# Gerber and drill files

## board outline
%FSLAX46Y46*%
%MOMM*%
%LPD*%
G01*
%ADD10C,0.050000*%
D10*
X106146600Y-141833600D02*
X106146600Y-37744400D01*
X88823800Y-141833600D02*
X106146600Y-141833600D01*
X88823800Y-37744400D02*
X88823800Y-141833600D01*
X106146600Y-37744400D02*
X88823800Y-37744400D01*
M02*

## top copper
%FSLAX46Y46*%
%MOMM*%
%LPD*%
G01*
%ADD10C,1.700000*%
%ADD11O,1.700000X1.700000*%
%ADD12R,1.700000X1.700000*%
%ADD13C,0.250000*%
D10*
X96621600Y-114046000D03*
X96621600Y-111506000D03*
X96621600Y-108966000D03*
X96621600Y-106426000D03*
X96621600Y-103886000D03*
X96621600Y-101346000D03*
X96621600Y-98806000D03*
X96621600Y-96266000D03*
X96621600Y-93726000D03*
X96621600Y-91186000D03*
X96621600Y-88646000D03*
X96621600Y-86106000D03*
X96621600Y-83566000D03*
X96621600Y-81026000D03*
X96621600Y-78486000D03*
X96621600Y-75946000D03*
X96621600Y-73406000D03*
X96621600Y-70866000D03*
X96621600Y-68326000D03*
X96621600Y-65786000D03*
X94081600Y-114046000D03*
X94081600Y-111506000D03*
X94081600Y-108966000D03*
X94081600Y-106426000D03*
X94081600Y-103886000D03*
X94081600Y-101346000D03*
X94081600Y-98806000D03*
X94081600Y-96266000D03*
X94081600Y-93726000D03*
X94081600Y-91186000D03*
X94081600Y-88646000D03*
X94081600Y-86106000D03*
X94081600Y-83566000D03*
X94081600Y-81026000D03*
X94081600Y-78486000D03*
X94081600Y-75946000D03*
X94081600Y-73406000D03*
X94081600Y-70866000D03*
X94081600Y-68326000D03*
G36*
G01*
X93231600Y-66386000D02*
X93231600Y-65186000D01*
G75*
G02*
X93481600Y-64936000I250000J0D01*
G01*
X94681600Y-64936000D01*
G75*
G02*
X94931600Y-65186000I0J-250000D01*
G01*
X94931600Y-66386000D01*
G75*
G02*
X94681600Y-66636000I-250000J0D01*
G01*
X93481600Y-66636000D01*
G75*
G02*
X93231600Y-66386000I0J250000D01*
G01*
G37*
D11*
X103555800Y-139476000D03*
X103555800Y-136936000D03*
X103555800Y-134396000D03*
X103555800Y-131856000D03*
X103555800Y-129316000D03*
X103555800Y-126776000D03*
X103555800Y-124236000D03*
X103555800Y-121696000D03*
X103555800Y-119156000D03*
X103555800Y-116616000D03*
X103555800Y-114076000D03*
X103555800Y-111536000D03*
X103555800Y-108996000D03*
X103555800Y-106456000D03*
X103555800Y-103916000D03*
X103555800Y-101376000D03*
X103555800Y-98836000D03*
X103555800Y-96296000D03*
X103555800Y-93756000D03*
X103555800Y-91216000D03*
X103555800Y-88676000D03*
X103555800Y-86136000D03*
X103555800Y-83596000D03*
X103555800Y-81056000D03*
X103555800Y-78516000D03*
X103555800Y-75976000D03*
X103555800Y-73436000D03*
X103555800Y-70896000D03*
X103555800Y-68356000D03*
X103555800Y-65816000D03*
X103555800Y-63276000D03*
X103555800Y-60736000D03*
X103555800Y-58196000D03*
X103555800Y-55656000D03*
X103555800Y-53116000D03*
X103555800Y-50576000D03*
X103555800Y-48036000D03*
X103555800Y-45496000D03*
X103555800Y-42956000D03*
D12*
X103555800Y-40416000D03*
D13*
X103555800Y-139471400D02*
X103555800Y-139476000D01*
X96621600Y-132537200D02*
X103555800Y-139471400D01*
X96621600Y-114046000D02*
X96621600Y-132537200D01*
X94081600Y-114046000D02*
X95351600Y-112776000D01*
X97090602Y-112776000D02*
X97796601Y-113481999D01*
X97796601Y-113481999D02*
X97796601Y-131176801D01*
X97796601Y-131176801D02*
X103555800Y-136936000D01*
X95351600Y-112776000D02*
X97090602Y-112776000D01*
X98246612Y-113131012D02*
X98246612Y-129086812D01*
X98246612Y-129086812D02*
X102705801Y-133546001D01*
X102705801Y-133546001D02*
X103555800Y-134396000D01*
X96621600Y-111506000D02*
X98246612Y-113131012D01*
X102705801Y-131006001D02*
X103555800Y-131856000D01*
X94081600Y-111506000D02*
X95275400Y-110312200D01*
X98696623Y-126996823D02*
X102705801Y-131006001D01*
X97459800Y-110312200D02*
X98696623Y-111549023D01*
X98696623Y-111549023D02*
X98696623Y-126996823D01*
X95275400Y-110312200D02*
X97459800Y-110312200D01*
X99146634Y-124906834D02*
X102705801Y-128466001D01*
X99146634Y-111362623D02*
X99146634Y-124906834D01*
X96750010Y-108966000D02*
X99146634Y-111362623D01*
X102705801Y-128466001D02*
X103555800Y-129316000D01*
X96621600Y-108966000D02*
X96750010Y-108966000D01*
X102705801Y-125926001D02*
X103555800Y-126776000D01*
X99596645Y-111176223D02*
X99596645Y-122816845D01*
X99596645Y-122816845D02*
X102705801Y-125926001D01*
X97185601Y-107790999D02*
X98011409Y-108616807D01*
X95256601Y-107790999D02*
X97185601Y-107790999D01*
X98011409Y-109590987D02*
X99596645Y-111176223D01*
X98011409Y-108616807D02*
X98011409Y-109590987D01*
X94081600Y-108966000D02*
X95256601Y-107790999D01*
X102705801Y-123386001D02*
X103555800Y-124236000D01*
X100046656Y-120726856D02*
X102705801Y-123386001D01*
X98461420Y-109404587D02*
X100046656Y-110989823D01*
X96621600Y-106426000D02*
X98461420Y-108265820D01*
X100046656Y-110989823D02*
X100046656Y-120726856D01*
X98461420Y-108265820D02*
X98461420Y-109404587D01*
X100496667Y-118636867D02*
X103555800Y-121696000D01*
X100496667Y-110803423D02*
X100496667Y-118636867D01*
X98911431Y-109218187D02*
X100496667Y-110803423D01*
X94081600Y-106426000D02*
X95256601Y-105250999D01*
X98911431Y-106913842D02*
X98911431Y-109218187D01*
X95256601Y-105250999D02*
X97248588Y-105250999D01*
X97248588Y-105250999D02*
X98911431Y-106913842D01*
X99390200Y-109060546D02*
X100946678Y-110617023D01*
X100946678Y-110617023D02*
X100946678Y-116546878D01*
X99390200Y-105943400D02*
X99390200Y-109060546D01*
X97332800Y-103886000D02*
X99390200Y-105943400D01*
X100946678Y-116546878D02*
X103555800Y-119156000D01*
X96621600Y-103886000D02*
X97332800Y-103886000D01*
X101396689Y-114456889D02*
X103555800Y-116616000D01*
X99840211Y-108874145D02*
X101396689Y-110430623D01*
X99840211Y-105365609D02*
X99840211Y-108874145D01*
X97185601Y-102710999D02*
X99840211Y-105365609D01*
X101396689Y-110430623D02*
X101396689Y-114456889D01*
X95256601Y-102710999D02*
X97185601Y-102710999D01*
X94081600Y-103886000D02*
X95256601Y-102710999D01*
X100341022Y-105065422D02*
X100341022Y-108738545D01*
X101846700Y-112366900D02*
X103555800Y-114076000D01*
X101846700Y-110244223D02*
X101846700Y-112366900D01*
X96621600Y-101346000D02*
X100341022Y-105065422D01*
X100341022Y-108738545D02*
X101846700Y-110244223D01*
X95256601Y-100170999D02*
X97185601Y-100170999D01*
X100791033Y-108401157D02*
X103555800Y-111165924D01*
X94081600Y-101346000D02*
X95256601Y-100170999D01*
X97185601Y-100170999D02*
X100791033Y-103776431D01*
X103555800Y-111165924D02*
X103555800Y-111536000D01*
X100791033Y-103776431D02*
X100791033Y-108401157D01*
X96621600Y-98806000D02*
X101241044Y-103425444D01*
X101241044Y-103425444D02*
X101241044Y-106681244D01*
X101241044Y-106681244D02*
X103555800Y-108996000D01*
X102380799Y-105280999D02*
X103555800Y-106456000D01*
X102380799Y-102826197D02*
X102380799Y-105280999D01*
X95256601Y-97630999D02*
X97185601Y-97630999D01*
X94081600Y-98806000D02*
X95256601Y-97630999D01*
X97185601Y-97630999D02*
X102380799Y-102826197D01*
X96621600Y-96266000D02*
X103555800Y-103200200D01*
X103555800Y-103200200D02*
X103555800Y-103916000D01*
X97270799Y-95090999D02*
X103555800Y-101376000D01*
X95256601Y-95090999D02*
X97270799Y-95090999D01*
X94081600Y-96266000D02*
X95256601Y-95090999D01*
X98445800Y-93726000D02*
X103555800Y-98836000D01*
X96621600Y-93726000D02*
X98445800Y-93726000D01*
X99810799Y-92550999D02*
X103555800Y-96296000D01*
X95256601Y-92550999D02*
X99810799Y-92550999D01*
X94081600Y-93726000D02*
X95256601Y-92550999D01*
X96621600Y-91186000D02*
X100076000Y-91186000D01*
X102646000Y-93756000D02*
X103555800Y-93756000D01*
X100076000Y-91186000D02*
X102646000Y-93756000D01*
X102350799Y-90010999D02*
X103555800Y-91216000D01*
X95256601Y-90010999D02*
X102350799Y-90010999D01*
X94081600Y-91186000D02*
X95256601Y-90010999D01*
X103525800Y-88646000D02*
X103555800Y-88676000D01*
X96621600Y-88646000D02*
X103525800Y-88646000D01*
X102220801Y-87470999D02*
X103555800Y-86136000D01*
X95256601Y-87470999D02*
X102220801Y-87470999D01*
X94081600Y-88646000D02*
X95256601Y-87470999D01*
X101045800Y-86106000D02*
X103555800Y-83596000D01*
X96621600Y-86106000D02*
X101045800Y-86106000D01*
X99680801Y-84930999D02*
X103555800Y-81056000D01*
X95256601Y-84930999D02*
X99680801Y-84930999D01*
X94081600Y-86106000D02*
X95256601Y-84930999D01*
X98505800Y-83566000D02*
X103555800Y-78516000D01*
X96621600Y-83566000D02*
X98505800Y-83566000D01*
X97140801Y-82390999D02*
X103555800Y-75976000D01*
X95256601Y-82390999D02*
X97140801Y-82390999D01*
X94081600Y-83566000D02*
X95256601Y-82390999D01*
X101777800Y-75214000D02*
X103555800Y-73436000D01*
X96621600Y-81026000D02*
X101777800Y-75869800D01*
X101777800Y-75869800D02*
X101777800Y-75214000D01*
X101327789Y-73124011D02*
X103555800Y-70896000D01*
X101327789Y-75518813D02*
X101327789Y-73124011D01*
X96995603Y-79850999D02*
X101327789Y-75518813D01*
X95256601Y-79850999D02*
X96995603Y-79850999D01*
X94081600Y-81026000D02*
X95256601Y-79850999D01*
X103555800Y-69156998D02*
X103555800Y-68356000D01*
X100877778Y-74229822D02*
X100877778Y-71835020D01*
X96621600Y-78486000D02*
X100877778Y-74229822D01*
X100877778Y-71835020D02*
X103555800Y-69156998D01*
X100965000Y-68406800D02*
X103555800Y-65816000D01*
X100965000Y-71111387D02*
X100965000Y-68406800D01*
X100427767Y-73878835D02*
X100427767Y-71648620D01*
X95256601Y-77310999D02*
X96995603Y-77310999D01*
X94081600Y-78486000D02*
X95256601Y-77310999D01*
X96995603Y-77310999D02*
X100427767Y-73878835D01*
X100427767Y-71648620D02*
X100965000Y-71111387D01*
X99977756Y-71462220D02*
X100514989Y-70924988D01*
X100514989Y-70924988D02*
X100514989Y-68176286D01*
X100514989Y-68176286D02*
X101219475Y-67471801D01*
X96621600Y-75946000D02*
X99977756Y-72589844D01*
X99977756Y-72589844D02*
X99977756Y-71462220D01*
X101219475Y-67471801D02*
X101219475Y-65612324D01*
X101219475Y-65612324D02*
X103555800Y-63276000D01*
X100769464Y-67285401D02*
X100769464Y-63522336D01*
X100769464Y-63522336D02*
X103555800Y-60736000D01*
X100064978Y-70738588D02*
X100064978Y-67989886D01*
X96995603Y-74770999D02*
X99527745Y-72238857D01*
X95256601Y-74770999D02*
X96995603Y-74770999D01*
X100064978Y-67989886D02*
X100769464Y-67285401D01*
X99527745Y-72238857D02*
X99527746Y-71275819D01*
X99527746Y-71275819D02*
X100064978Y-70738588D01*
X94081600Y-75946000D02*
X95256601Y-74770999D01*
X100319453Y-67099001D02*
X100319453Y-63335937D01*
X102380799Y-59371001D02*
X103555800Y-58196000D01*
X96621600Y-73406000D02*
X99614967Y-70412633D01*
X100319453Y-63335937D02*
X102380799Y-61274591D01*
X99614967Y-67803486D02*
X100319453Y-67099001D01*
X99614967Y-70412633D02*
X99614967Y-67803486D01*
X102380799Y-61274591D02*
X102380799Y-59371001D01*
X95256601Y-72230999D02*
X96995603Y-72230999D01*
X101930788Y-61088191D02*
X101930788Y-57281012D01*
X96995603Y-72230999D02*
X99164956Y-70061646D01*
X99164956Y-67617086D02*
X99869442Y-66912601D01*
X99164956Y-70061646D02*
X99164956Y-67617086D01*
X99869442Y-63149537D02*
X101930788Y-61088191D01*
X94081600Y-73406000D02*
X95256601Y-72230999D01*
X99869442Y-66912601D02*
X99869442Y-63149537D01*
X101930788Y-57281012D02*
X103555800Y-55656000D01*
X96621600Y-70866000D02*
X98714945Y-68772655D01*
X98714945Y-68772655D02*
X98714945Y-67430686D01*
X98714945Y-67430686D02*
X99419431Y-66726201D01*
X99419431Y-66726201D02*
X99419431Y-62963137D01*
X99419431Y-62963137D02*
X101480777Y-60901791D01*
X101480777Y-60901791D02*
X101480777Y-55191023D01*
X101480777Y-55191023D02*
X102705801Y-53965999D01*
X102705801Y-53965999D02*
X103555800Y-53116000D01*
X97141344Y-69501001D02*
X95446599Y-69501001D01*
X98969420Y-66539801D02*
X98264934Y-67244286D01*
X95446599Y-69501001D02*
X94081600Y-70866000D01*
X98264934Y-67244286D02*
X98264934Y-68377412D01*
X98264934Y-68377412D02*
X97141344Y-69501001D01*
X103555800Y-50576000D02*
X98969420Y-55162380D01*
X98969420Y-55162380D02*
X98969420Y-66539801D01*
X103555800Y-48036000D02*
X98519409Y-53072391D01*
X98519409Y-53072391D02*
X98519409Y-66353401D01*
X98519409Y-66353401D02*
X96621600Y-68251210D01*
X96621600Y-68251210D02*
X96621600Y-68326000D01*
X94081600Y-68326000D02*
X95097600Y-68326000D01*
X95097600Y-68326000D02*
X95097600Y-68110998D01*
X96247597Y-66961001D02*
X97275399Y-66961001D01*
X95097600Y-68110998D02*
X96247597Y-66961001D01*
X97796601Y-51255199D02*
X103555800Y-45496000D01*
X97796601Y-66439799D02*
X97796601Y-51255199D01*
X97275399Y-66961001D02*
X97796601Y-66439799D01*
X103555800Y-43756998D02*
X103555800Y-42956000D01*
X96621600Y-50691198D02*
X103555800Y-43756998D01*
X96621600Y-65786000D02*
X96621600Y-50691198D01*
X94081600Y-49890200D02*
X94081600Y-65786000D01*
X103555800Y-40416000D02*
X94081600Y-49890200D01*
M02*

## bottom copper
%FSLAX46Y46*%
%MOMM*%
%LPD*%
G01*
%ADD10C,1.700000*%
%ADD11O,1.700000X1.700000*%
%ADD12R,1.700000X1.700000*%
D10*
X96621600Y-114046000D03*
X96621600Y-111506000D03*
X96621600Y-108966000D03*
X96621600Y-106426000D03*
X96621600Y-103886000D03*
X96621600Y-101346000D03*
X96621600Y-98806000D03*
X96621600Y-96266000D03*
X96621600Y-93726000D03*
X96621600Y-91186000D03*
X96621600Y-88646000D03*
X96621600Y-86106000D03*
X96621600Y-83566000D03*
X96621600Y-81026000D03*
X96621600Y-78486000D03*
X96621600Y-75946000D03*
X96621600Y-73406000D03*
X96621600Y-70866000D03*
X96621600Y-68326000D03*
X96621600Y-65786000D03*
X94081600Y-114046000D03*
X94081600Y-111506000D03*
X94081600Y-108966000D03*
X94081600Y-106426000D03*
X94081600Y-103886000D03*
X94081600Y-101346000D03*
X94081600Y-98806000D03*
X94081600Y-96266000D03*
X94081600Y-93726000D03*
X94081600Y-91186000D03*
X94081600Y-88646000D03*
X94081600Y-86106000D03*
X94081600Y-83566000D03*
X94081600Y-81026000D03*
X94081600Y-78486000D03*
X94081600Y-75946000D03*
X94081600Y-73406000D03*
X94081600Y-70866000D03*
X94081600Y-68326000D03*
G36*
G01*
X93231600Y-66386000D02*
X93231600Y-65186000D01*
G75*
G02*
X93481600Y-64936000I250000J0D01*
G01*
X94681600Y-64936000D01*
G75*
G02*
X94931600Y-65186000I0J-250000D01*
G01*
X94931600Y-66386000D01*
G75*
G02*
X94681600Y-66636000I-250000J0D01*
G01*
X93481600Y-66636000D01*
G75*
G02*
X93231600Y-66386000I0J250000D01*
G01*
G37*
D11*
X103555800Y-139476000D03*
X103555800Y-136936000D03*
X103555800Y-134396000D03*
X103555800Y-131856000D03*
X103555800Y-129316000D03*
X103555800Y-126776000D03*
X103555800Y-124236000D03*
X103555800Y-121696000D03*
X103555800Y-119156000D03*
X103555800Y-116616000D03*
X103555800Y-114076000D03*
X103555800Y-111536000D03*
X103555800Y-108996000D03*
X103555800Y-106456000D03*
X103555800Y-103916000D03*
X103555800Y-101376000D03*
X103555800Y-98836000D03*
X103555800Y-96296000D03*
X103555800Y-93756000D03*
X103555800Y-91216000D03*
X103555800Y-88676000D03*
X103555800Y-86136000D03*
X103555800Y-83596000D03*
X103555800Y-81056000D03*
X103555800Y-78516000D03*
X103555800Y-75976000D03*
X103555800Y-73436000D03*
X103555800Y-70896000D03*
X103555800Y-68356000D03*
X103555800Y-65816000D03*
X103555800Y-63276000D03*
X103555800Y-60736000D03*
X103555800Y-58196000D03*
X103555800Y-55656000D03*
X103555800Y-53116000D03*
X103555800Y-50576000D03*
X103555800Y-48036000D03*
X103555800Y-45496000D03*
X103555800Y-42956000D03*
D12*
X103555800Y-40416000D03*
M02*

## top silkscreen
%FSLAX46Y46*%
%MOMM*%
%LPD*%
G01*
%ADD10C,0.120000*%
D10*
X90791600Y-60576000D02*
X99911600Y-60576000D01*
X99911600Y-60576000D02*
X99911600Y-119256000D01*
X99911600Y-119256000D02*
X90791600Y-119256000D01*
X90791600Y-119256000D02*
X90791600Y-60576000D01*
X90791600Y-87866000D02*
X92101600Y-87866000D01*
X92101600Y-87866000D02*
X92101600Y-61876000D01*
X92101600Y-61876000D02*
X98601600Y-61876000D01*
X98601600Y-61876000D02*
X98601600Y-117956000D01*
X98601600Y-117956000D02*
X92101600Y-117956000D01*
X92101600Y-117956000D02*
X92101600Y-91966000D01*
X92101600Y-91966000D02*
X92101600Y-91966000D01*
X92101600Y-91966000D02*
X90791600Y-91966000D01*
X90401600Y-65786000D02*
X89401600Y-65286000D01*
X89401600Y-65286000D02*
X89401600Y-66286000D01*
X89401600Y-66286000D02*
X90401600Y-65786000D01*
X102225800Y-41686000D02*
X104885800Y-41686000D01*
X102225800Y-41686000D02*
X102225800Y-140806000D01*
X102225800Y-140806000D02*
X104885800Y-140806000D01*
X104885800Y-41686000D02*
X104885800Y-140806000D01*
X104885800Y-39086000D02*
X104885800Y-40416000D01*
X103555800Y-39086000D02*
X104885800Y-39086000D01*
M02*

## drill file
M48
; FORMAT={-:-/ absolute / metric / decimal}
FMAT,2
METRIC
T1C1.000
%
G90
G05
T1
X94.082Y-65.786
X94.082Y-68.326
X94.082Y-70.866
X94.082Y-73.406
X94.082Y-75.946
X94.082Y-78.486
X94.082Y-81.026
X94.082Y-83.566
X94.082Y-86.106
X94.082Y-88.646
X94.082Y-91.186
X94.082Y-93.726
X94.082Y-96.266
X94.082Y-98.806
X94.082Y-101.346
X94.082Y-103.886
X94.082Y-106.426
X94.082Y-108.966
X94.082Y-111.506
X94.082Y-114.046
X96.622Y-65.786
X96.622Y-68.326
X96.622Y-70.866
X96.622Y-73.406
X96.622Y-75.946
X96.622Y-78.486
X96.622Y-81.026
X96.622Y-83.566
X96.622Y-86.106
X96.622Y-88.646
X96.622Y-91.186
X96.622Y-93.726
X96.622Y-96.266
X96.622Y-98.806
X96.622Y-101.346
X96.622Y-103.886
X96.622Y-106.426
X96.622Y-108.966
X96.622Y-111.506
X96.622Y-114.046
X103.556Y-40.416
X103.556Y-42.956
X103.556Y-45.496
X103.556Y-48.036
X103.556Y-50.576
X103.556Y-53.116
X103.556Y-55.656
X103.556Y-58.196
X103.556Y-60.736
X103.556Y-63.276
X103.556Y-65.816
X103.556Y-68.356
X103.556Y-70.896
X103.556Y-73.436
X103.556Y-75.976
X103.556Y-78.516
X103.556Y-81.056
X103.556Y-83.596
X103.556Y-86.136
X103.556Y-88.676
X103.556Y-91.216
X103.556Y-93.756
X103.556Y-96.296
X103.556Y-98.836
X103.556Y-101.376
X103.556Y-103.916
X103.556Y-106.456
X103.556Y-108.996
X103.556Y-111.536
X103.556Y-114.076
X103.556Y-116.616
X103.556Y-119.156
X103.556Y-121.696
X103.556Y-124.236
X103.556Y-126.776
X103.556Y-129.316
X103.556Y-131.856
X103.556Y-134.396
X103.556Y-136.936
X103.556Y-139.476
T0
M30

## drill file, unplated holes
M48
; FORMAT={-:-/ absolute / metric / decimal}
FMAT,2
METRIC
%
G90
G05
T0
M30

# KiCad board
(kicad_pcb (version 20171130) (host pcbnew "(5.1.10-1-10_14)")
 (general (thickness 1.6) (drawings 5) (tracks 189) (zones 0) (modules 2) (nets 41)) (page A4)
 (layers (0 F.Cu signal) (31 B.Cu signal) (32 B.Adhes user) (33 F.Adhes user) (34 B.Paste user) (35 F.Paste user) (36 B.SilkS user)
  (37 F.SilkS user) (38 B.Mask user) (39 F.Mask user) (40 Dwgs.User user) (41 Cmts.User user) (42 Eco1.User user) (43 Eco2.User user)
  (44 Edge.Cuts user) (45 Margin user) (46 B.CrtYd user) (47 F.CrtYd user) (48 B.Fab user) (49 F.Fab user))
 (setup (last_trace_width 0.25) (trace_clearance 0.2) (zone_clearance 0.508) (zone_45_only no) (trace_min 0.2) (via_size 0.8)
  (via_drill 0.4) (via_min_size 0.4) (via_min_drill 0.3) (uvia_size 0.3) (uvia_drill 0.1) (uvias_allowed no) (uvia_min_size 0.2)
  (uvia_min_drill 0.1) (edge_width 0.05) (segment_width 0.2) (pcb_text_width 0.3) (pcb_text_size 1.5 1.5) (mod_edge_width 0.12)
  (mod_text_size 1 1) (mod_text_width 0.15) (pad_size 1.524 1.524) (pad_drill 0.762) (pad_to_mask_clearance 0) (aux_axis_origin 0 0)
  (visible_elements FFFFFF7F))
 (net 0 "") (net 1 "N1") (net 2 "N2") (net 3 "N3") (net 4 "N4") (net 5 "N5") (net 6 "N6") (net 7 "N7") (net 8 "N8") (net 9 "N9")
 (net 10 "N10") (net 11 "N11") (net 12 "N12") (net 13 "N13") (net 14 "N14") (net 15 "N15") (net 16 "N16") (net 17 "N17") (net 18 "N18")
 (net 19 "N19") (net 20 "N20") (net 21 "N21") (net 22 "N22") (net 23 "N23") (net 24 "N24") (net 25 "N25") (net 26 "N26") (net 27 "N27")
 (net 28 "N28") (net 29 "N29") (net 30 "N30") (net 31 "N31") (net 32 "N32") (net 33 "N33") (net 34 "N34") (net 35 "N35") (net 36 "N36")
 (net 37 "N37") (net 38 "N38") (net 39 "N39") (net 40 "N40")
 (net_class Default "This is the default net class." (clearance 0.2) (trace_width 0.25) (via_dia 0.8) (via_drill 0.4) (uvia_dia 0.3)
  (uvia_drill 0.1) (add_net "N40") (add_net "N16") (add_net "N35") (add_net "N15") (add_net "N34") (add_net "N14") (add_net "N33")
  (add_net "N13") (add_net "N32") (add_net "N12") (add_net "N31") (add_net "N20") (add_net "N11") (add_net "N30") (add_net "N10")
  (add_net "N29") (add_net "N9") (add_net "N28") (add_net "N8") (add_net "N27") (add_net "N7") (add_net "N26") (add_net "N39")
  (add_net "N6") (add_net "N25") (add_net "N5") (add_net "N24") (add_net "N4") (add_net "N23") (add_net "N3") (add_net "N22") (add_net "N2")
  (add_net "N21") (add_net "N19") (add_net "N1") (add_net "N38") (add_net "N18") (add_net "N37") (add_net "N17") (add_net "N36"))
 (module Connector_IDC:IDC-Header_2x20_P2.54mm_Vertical (layer F.Cu) (at 94.0816 65.786)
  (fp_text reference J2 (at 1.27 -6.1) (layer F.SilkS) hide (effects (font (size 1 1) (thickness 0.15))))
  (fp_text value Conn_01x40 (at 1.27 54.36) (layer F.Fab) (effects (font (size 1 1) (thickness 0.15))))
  (fp_line (start -3.29 -5.21) (end 5.83 -5.21) (layer F.SilkS) (width 0.12))
  (fp_line (start 5.83 -5.21) (end 5.83 53.47) (layer F.SilkS) (width 0.12))
  (fp_line (start 5.83 53.47) (end -3.29 53.47) (layer F.SilkS) (width 0.12))
  (fp_line (start -3.29 53.47) (end -3.29 -5.21) (layer F.SilkS) (width 0.12))
  (fp_line (start -3.29 22.08) (end -1.98 22.08) (layer F.SilkS) (width 0.12))
  (fp_line (start -1.98 22.08) (end -1.98 -3.91) (layer F.SilkS) (width 0.12))
  (fp_line (start -1.98 -3.91) (end 4.52 -3.91) (layer F.SilkS) (width 0.12))
  (fp_line (start 4.52 -3.91) (end 4.52 52.17) (layer F.SilkS) (width 0.12))
  (fp_line (start 4.52 52.17) (end -1.98 52.17) (layer F.SilkS) (width 0.12))
  (fp_line (start -1.98 52.17) (end -1.98 26.18) (layer F.SilkS) (width 0.12))
  (fp_line (start -1.98 26.18) (end -1.98 26.18) (layer F.SilkS) (width 0.12))
  (fp_line (start -1.98 26.18) (end -3.29 26.18) (layer F.SilkS) (width 0.12))
  (fp_line (start -3.68 0) (end -4.68 -0.5) (layer F.SilkS) (width 0.12))
  (fp_line (start -4.68 -0.5) (end -4.68 0.5) (layer F.SilkS) (width 0.12))
  (fp_line (start -4.68 0.5) (end -3.68 0) (layer F.SilkS) (width 0.12))
  (pad 40 thru_hole circle (at 2.54 48.26) (size 1.7 1.7) (drill 1) (layers *.Cu *.Mask) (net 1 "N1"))
  (pad 38 thru_hole circle (at 2.54 45.72) (size 1.7 1.7) (drill 1) (layers *.Cu *.Mask) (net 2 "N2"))
  (pad 36 thru_hole circle (at 2.54 43.18) (size 1.7 1.7) (drill 1) (layers *.Cu *.Mask) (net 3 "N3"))
  (pad 34 thru_hole circle (at 2.54 40.64) (size 1.7 1.7) (drill 1) (layers *.Cu *.Mask) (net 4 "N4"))
  (pad 32 thru_hole circle (at 2.54 38.1) (size 1.7 1.7) (drill 1) (layers *.Cu *.Mask) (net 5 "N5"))
  (pad 30 thru_hole circle (at 2.54 35.56) (size 1.7 1.7) (drill 1) (layers *.Cu *.Mask) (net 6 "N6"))
  (pad 28 thru_hole circle (at 2.54 33.02) (size 1.7 1.7) (drill 1) (layers *.Cu *.Mask) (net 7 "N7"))
  (pad 26 thru_hole circle (at 2.54 30.48) (size 1.7 1.7) (drill 1) (layers *.Cu *.Mask) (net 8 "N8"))
  (pad 24 thru_hole circle (at 2.54 27.94) (size 1.7 1.7) (drill 1) (layers *.Cu *.Mask) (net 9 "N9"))
  (pad 22 thru_hole circle (at 2.54 25.4) (size 1.7 1.7) (drill 1) (layers *.Cu *.Mask) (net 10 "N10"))
  (pad 20 thru_hole circle (at 2.54 22.86) (size 1.7 1.7) (drill 1) (layers *.Cu *.Mask) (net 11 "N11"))
  (pad 18 thru_hole circle (at 2.54 20.32) (size 1.7 1.7) (drill 1) (layers *.Cu *.Mask) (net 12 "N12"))
  (pad 16 thru_hole circle (at 2.54 17.78) (size 1.7 1.7) (drill 1) (layers *.Cu *.Mask) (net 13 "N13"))
  (pad 14 thru_hole circle (at 2.54 15.24) (size 1.7 1.7) (drill 1) (layers *.Cu *.Mask) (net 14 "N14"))
  (pad 12 thru_hole circle (at 2.54 12.7) (size 1.7 1.7) (drill 1) (layers *.Cu *.Mask) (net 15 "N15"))
  (pad 10 thru_hole circle (at 2.54 10.16) (size 1.7 1.7) (drill 1) (layers *.Cu *.Mask) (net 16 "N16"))
  (pad 8 thru_hole circle (at 2.54 7.62) (size 1.7 1.7) (drill 1) (layers *.Cu *.Mask) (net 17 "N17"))
  (pad 6 thru_hole circle (at 2.54 5.08) (size 1.7 1.7) (drill 1) (layers *.Cu *.Mask) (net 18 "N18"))
  (pad 4 thru_hole circle (at 2.54 2.54) (size 1.7 1.7) (drill 1) (layers *.Cu *.Mask) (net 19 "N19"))
  (pad 2 thru_hole circle (at 2.54 0) (size 1.7 1.7) (drill 1) (layers *.Cu *.Mask) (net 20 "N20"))
  (pad 39 thru_hole circle (at 0 48.26) (size 1.7 1.7) (drill 1) (layers *.Cu *.Mask) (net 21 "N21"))
  (pad 37 thru_hole circle (at 0 45.72) (size 1.7 1.7) (drill 1) (layers *.Cu *.Mask) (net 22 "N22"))
  (pad 35 thru_hole circle (at 0 43.18) (size 1.7 1.7) (drill 1) (layers *.Cu *.Mask) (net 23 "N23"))
  (pad 33 thru_hole circle (at 0 40.64) (size 1.7 1.7) (drill 1) (layers *.Cu *.Mask) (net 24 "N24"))
  (pad 31 thru_hole circle (at 0 38.1) (size 1.7 1.7) (drill 1) (layers *.Cu *.Mask) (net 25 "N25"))
  (pad 29 thru_hole circle (at 0 35.56) (size 1.7 1.7) (drill 1) (layers *.Cu *.Mask) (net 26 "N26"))
  (pad 27 thru_hole circle (at 0 33.02) (size 1.7 1.7) (drill 1) (layers *.Cu *.Mask) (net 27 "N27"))
  (pad 25 thru_hole circle (at 0 30.48) (size 1.7 1.7) (drill 1) (layers *.Cu *.Mask) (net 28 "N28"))
  (pad 23 thru_hole circle (at 0 27.94) (size 1.7 1.7) (drill 1) (layers *.Cu *.Mask) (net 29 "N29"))
  (pad 21 thru_hole circle (at 0 25.4) (size 1.7 1.7) (drill 1) (layers *.Cu *.Mask) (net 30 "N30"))
  (pad 19 thru_hole circle (at 0 22.86) (size 1.7 1.7) (drill 1) (layers *.Cu *.Mask) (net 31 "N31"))
  (pad 17 thru_hole circle (at 0 20.32) (size 1.7 1.7) (drill 1) (layers *.Cu *.Mask) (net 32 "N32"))
  (pad 15 thru_hole circle (at 0 17.78) (size 1.7 1.7) (drill 1) (layers *.Cu *.Mask) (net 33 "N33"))
  (pad 13 thru_hole circle (at 0 15.24) (size 1.7 1.7) (drill 1) (layers *.Cu *.Mask) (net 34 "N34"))
  (pad 11 thru_hole circle (at 0 12.7) (size 1.7 1.7) (drill 1) (layers *.Cu *.Mask) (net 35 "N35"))
  (pad 9 thru_hole circle (at 0 10.16) (size 1.7 1.7) (drill 1) (layers *.Cu *.Mask) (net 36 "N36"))
  (pad 7 thru_hole circle (at 0 7.62) (size 1.7 1.7) (drill 1) (layers *.Cu *.Mask) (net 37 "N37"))
  (pad 5 thru_hole circle (at 0 5.08) (size 1.7 1.7) (drill 1) (layers *.Cu *.Mask) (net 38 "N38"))
  (pad 3 thru_hole circle (at 0 2.54) (size 1.7 1.7) (drill 1) (layers *.Cu *.Mask) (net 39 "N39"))
  (pad 1 thru_hole roundrect (at 0 0) (size 1.7 1.7) (drill 1) (layers *.Cu *.Mask) (roundrect_rratio 0.1470588235294118) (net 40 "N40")))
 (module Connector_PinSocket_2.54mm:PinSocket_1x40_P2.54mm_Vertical (layer F.Cu) (at 103.5558 40.416)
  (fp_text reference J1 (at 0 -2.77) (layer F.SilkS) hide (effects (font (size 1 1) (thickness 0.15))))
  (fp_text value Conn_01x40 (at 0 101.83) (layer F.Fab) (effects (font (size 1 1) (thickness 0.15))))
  (fp_line (start -1.33 1.27) (end 1.33 1.27) (layer F.SilkS) (width 0.12))
  (fp_line (start -1.33 1.27) (end -1.33 100.39) (layer F.SilkS) (width 0.12))
  (fp_line (start -1.33 100.39) (end 1.33 100.39) (layer F.SilkS) (width 0.12))
  (fp_line (start 1.33 1.27) (end 1.33 100.39) (layer F.SilkS) (width 0.12))
  (fp_line (start 1.33 -1.33) (end 1.33 0) (layer F.SilkS) (width 0.12))
  (fp_line (start 0 -1.33) (end 1.33 -1.33) (layer F.SilkS) (width 0.12))
  (pad 40 thru_hole oval (at 0 99.06) (size 1.7 1.7) (drill 1) (layers *.Cu *.Mask) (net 1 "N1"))
  (pad 39 thru_hole oval (at 0 96.52) (size 1.7 1.7) (drill 1) (layers *.Cu *.Mask) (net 21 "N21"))
  (pad 38 thru_hole oval (at 0 93.98) (size 1.7 1.7) (drill 1) (layers *.Cu *.Mask) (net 2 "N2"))
  (pad 37 thru_hole oval (at 0 91.44) (size 1.7 1.7) (drill 1) (layers *.Cu *.Mask) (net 22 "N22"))
  (pad 36 thru_hole oval (at 0 88.9) (size 1.7 1.7) (drill 1) (layers *.Cu *.Mask) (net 3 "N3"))
  (pad 35 thru_hole oval (at 0 86.36) (size 1.7 1.7) (drill 1) (layers *.Cu *.Mask) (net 23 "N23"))
  (pad 34 thru_hole oval (at 0 83.82) (size 1.7 1.7) (drill 1) (layers *.Cu *.Mask) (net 4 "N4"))
  (pad 33 thru_hole oval (at 0 81.28) (size 1.7 1.7) (drill 1) (layers *.Cu *.Mask) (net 24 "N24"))
  (pad 32 thru_hole oval (at 0 78.74) (size 1.7 1.7) (drill 1) (layers *.Cu *.Mask) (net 5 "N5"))
  (pad 31 thru_hole oval (at 0 76.2) (size 1.7 1.7) (drill 1) (layers *.Cu *.Mask) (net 25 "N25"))
  (pad 30 thru_hole oval (at 0 73.66) (size 1.7 1.7) (drill 1) (layers *.Cu *.Mask) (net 6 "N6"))
  (pad 29 thru_hole oval (at 0 71.12) (size 1.7 1.7) (drill 1) (layers *.Cu *.Mask) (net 26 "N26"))
  (pad 28 thru_hole oval (at 0 68.58) (size 1.7 1.7) (drill 1) (layers *.Cu *.Mask) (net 7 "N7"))
  (pad 27 thru_hole oval (at 0 66.04) (size 1.7 1.7) (drill 1) (layers *.Cu *.Mask) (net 27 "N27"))
  (pad 26 thru_hole oval (at 0 63.5) (size 1.7 1.7) (drill 1) (layers *.Cu *.Mask) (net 8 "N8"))
  (pad 25 thru_hole oval (at 0 60.96) (size 1.7 1.7) (drill 1) (layers *.Cu *.Mask) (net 28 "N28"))
  (pad 24 thru_hole oval (at 0 58.42) (size 1.7 1.7) (drill 1) (layers *.Cu *.Mask) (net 9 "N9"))
  (pad 23 thru_hole oval (at 0 55.88) (size 1.7 1.7) (drill 1) (layers *.Cu *.Mask) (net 29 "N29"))
  (pad 22 thru_hole oval (at 0 53.34) (size 1.7 1.7) (drill 1) (layers *.Cu *.Mask) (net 10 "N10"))
  (pad 21 thru_hole oval (at 0 50.8) (size 1.7 1.7) (drill 1) (layers *.Cu *.Mask) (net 30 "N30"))
  (pad 20 thru_hole oval (at 0 48.26) (size 1.7 1.7) (drill 1) (layers *.Cu *.Mask) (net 11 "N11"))
  (pad 19 thru_hole oval (at 0 45.72) (size 1.7 1.7) (drill 1) (layers *.Cu *.Mask) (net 31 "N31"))
  (pad 18 thru_hole oval (at 0 43.18) (size 1.7 1.7) (drill 1) (layers *.Cu *.Mask) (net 12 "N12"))
  (pad 17 thru_hole oval (at 0 40.64) (size 1.7 1.7) (drill 1) (layers *.Cu *.Mask) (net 32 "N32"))
  (pad 16 thru_hole oval (at 0 38.1) (size 1.7 1.7) (drill 1) (layers *.Cu *.Mask) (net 13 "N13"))
  (pad 15 thru_hole oval (at 0 35.56) (size 1.7 1.7) (drill 1) (layers *.Cu *.Mask) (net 33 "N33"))
  (pad 14 thru_hole oval (at 0 33.02) (size 1.7 1.7) (drill 1) (layers *.Cu *.Mask) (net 14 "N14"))
  (pad 13 thru_hole oval (at 0 30.48) (size 1.7 1.7) (drill 1) (layers *.Cu *.Mask) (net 34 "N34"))
  (pad 12 thru_hole oval (at 0 27.94) (size 1.7 1.7) (drill 1) (layers *.Cu *.Mask) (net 15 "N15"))
  (pad 11 thru_hole oval (at 0 25.4) (size 1.7 1.7) (drill 1) (layers *.Cu *.Mask) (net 35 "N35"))
  (pad 10 thru_hole oval (at 0 22.86) (size 1.7 1.7) (drill 1) (layers *.Cu *.Mask) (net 16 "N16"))
  (pad 9 thru_hole oval (at 0 20.32) (size 1.7 1.7) (drill 1) (layers *.Cu *.Mask) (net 36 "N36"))
  (pad 8 thru_hole oval (at 0 17.78) (size 1.7 1.7) (drill 1) (layers *.Cu *.Mask) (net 17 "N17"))
  (pad 7 thru_hole oval (at 0 15.24) (size 1.7 1.7) (drill 1) (layers *.Cu *.Mask) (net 37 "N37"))
  (pad 6 thru_hole oval (at 0 12.7) (size 1.7 1.7) (drill 1) (layers *.Cu *.Mask) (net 18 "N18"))
  (pad 5 thru_hole oval (at 0 10.16) (size 1.7 1.7) (drill 1) (layers *.Cu *.Mask) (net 38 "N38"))
  (pad 4 thru_hole oval (at 0 7.62) (size 1.7 1.7) (drill 1) (layers *.Cu *.Mask) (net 19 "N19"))
  (pad 3 thru_hole oval (at 0 5.08) (size 1.7 1.7) (drill 1) (layers *.Cu *.Mask) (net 39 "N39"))
  (pad 2 thru_hole oval (at 0 2.54) (size 1.7 1.7) (drill 1) (layers *.Cu *.Mask) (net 20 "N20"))
  (pad 1 thru_hole rect (at 0 0) (size 1.7 1.7) (drill 1) (layers *.Cu *.Mask) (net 40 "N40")))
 (gr_line (start 106.1466 141.8336) (end 106.1466 37.7444) (layer Edge.Cuts) (width 0.05))
 (gr_line (start 88.8238 141.8336) (end 106.1466 141.8336) (layer Edge.Cuts) (width 0.05))
 (gr_line (start 88.8238 37.7444) (end 88.8238 141.8336) (layer Edge.Cuts) (width 0.05))
 (gr_line (start 106.1466 37.7444) (end 88.8238 37.7444) (layer Edge.Cuts) (width 0.05))
 (segment (start 103.5558 139.4714) (end 103.5558 139.476) (width 0.25) (layer F.Cu) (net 1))
 (segment (start 96.6216 132.5372) (end 103.5558 139.4714) (width 0.25) (layer F.Cu) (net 1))
 (segment (start 96.6216 114.046) (end 96.6216 132.5372) (width 0.25) (layer F.Cu) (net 1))
 (segment (start 94.0816 114.046) (end 95.3516 112.776) (width 0.25) (layer F.Cu) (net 21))
 (segment (start 97.090602 112.776) (end 97.796601 113.481999) (width 0.25) (layer F.Cu) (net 21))
 (segment (start 97.796601 113.481999) (end 97.796601 131.176801) (width 0.25) (layer F.Cu) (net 21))
 (segment (start 97.796601 131.176801) (end 103.5558 136.936) (width 0.25) (layer F.Cu) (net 21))
 (segment (start 95.3516 112.776) (end 97.090602 112.776) (width 0.25) (layer F.Cu) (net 21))
 (segment (start 98.246612 113.131012) (end 98.246612 129.086812) (width 0.25) (layer F.Cu) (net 2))
 (segment (start 98.246612 129.086812) (end 102.705801 133.546001) (width 0.25) (layer F.Cu) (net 2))
 (segment (start 102.705801 133.546001) (end 103.5558 134.396) (width 0.25) (layer F.Cu) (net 2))
 (segment (start 96.6216 111.506) (end 98.246612 113.131012) (width 0.25) (layer F.Cu) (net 2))
 (segment (start 102.705801 131.006001) (end 103.5558 131.856) (width 0.25) (layer F.Cu) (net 22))
 (segment (start 94.0816 111.506) (end 95.2754 110.3122) (width 0.25) (layer F.Cu) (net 22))
 (segment (start 98.696623 126.996823) (end 102.705801 131.006001) (width 0.25) (layer F.Cu) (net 22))
 (segment (start 97.4598 110.3122) (end 98.696623 111.549023) (width 0.25) (layer F.Cu) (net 22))
 (segment (start 98.696623 111.549023) (end 98.696623 126.996823) (width 0.25) (layer F.Cu) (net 22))
 (segment (start 95.2754 110.3122) (end 97.4598 110.3122) (width 0.25) (layer F.Cu) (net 22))
 (segment (start 99.146634 124.906834) (end 102.705801 128.466001) (width 0.25) (layer F.Cu) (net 3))
 (segment (start 99.146634 111.362623) (end 99.146634 124.906834) (width 0.25) (layer F.Cu) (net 3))
 (segment (start 96.75001 108.966) (end 99.146634 111.362623) (width 0.25) (layer F.Cu) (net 3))
 (segment (start 102.705801 128.466001) (end 103.5558 129.316) (width 0.25) (layer F.Cu) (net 3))
 (segment (start 96.6216 108.966) (end 96.75001 108.966) (width 0.25) (layer F.Cu) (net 3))
 (segment (start 102.705801 125.926001) (end 103.5558 126.776) (width 0.25) (layer F.Cu) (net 23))
 (segment (start 99.596645 111.176223) (end 99.596645 122.816845) (width 0.25) (layer F.Cu) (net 23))
 (segment (start 99.596645 122.816845) (end 102.705801 125.926001) (width 0.25) (layer F.Cu) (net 23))
 (segment (start 97.185601 107.790999) (end 98.011409 108.616807) (width 0.25) (layer F.Cu) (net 23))
 (segment (start 95.256601 107.790999) (end 97.185601 107.790999) (width 0.25) (layer F.Cu) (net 23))
 (segment (start 98.011409 109.590987) (end 99.596645 111.176223) (width 0.25) (layer F.Cu) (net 23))
 (segment (start 98.011409 108.616807) (end 98.011409 109.590987) (width 0.25) (layer F.Cu) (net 23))
 (segment (start 94.0816 108.966) (end 95.256601 107.790999) (width 0.25) (layer F.Cu) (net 23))
 (segment (start 102.705801 123.386001) (end 103.5558 124.236) (width 0.25) (layer F.Cu) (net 4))
 (segment (start 100.046656 120.726856) (end 102.705801 123.386001) (width 0.25) (layer F.Cu) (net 4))
 (segment (start 98.46142 109.404587) (end 100.046656 110.989823) (width 0.25) (layer F.Cu) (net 4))
 (segment (start 96.6216 106.426) (end 98.46142 108.26582) (width 0.25) (layer F.Cu) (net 4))
 (segment (start 100.046656 110.989823) (end 100.046656 120.726856) (width 0.25) (layer F.Cu) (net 4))
 (segment (start 98.46142 108.26582) (end 98.46142 109.404587) (width 0.25) (layer F.Cu) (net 4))
 (segment (start 100.496667 118.636867) (end 103.5558 121.696) (width 0.25) (layer F.Cu) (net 24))
 (segment (start 100.496667 110.803423) (end 100.496667 118.636867) (width 0.25) (layer F.Cu) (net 24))
 (segment (start 98.911431 109.218187) (end 100.496667 110.803423) (width 0.25) (layer F.Cu) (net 24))
 (segment (start 94.0816 106.426) (end 95.256601 105.250999) (width 0.25) (layer F.Cu) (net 24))
 (segment (start 98.911431 106.913842) (end 98.911431 109.218187) (width 0.25) (layer F.Cu) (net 24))
 (segment (start 95.256601 105.250999) (end 97.248588 105.250999) (width 0.25) (layer F.Cu) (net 24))
 (segment (start 97.248588 105.250999) (end 98.911431 106.913842) (width 0.25) (layer F.Cu) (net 24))
 (segment (start 99.3902 109.060546) (end 100.946678 110.617023) (width 0.25) (layer F.Cu) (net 5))
 (segment (start 100.946678 110.617023) (end 100.946678 116.546878) (width 0.25) (layer F.Cu) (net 5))
 (segment (start 99.3902 105.9434) (end 99.3902 109.060546) (width 0.25) (layer F.Cu) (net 5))
 (segment (start 97.3328 103.886) (end 99.3902 105.9434) (width 0.25) (layer F.Cu) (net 5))
 (segment (start 100.946678 116.546878) (end 103.5558 119.156) (width 0.25) (layer F.Cu) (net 5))
 (segment (start 96.6216 103.886) (end 97.3328 103.886) (width 0.25) (layer F.Cu) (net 5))
 (segment (start 101.396689 114.456889) (end 103.5558 116.616) (width 0.25) (layer F.Cu) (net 25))
 (segment (start 99.840211 108.874145) (end 101.396689 110.430623) (width 0.25) (layer F.Cu) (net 25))
 (segment (start 99.840211 105.365609) (end 99.840211 108.874145) (width 0.25) (layer F.Cu) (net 25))
 (segment (start 97.185601 102.710999) (end 99.840211 105.365609) (width 0.25) (layer F.Cu) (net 25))
 (segment (start 101.396689 110.430623) (end 101.396689 114.456889) (width 0.25) (layer F.Cu) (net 25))
 (segment (start 95.256601 102.710999) (end 97.185601 102.710999) (width 0.25) (layer F.Cu) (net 25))
 (segment (start 94.0816 103.886) (end 95.256601 102.710999) (width 0.25) (layer F.Cu) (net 25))
 (segment (start 100.341022 105.065422) (end 100.341022 108.738545) (width 0.25) (layer F.Cu) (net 6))
 (segment (start 101.8467 112.3669) (end 103.5558 114.076) (width 0.25) (layer F.Cu) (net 6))
 (segment (start 101.8467 110.244223) (end 101.8467 112.3669) (width 0.25) (layer F.Cu) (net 6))
 (segment (start 96.6216 101.346) (end 100.341022 105.065422) (width 0.25) (layer F.Cu) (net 6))
 (segment (start 100.341022 108.738545) (end 101.8467 110.244223) (width 0.25) (layer F.Cu) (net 6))
 (segment (start 95.256601 100.170999) (end 97.185601 100.170999) (width 0.25) (layer F.Cu) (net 26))
 (segment (start 100.791033 108.401157) (end 103.5558 111.165924) (width 0.25) (layer F.Cu) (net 26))
 (segment (start 94.0816 101.346) (end 95.256601 100.170999) (width 0.25) (layer F.Cu) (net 26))
 (segment (start 97.185601 100.170999) (end 100.791033 103.776431) (width 0.25) (layer F.Cu) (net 26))
 (segment (start 103.5558 111.165924) (end 103.5558 111.536) (width 0.25) (layer F.Cu) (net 26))
 (segment (start 100.791033 103.776431) (end 100.791033 108.401157) (width 0.25) (layer F.Cu) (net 26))
 (segment (start 96.6216 98.806) (end 101.241044 103.425444) (width 0.25) (layer F.Cu) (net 7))
 (segment (start 101.241044 103.425444) (end 101.241044 106.681244) (width 0.25) (layer F.Cu) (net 7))
 (segment (start 101.241044 106.681244) (end 103.5558 108.996) (width 0.25) (layer F.Cu) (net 7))
 (segment (start 102.380799 105.280999) (end 103.5558 106.456) (width 0.25) (layer F.Cu) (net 27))
 (segment (start 102.380799 102.826197) (end 102.380799 105.280999) (width 0.25) (layer F.Cu) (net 27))
 (segment (start 95.256601 97.630999) (end 97.185601 97.630999) (width 0.25) (layer F.Cu) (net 27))
 (segment (start 94.0816 98.806) (end 95.256601 97.630999) (width 0.25) (layer F.Cu) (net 27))
 (segment (start 97.185601 97.630999) (end 102.380799 102.826197) (width 0.25) (layer F.Cu) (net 27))
 (segment (start 96.6216 96.266) (end 103.5558 103.2002) (width 0.25) (layer F.Cu) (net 8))
 (segment (start 103.5558 103.2002) (end 103.5558 103.916) (width 0.25) (layer F.Cu) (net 8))
 (segment (start 97.270799 95.090999) (end 103.5558 101.376) (width 0.25) (layer F.Cu) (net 28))
 (segment (start 95.256601 95.090999) (end 97.270799 95.090999) (width 0.25) (layer F.Cu) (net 28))
 (segment (start 94.0816 96.266) (end 95.256601 95.090999) (width 0.25) (layer F.Cu) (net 28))
 (segment (start 98.4458 93.726) (end 103.5558 98.836) (width 0.25) (layer F.Cu) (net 9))
 (segment (start 96.6216 93.726) (end 98.4458 93.726) (width 0.25) (layer F.Cu) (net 9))
 (segment (start 99.810799 92.550999) (end 103.5558 96.296) (width 0.25) (layer F.Cu) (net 29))
 (segment (start 95.256601 92.550999) (end 99.810799 92.550999) (width 0.25) (layer F.Cu) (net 29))
 (segment (start 94.0816 93.726) (end 95.256601 92.550999) (width 0.25) (layer F.Cu) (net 29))
 (segment (start 96.6216 91.186) (end 100.076 91.186) (width 0.25) (layer F.Cu) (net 10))
 (segment (start 102.646 93.756) (end 103.5558 93.756) (width 0.25) (layer F.Cu) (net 10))
 (segment (start 100.076 91.186) (end 102.646 93.756) (width 0.25) (layer F.Cu) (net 10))
 (segment (start 102.350799 90.010999) (end 103.5558 91.216) (width 0.25) (layer F.Cu) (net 30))
 (segment (start 95.256601 90.010999) (end 102.350799 90.010999) (width 0.25) (layer F.Cu) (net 30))
 (segment (start 94.0816 91.186) (end 95.256601 90.010999) (width 0.25) (layer F.Cu) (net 30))
 (segment (start 103.5258 88.646) (end 103.5558 88.676) (width 0.25) (layer F.Cu) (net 11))
 (segment (start 96.6216 88.646) (end 103.5258 88.646) (width 0.25) (layer F.Cu) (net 11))
 (segment (start 102.220801 87.470999) (end 103.5558 86.136) (width 0.25) (layer F.Cu) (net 31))
 (segment (start 95.256601 87.470999) (end 102.220801 87.470999) (width 0.25) (layer F.Cu) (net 31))
 (segment (start 94.0816 88.646) (end 95.256601 87.470999) (width 0.25) (layer F.Cu) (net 31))
 (segment (start 101.0458 86.106) (end 103.5558 83.596) (width 0.25) (layer F.Cu) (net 12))
 (segment (start 96.6216 86.106) (end 101.0458 86.106) (width 0.25) (layer F.Cu) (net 12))
 (segment (start 99.680801 84.930999) (end 103.5558 81.056) (width 0.25) (layer F.Cu) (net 32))
 (segment (start 95.256601 84.930999) (end 99.680801 84.930999) (width 0.25) (layer F.Cu) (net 32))
 (segment (start 94.0816 86.106) (end 95.256601 84.930999) (width 0.25) (layer F.Cu) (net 32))
 (segment (start 98.5058 83.566) (end 103.5558 78.516) (width 0.25) (layer F.Cu) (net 13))
 (segment (start 96.6216 83.566) (end 98.5058 83.566) (width 0.25) (layer F.Cu) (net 13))
 (segment (start 97.140801 82.390999) (end 103.5558 75.976) (width 0.25) (layer F.Cu) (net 33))
 (segment (start 95.256601 82.390999) (end 97.140801 82.390999) (width 0.25) (layer F.Cu) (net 33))
 (segment (start 94.0816 83.566) (end 95.256601 82.390999) (width 0.25) (layer F.Cu) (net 33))
 (segment (start 101.7778 75.214) (end 103.5558 73.436) (width 0.25) (layer F.Cu) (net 14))
 (segment (start 96.6216 81.026) (end 101.7778 75.8698) (width 0.25) (layer F.Cu) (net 14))
 (segment (start 101.7778 75.8698) (end 101.7778 75.214) (width 0.25) (layer F.Cu) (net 14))
 (segment (start 101.327789 73.124011) (end 103.5558 70.896) (width 0.25) (layer F.Cu) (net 34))
 (segment (start 101.327789 75.518813) (end 101.327789 73.124011) (width 0.25) (layer F.Cu) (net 34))
 (segment (start 96.995603 79.850999) (end 101.327789 75.518813) (width 0.25) (layer F.Cu) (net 34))
 (segment (start 95.256601 79.850999) (end 96.995603 79.850999) (width 0.25) (layer F.Cu) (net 34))
 (segment (start 94.0816 81.026) (end 95.256601 79.850999) (width 0.25) (layer F.Cu) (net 34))
 (segment (start 103.5558 69.156998) (end 103.5558 68.356) (width 0.25) (layer F.Cu) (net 15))
 (segment (start 100.877778 74.229822) (end 100.877778 71.83502) (width 0.25) (layer F.Cu) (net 15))
 (segment (start 96.6216 78.486) (end 100.877778 74.229822) (width 0.25) (layer F.Cu) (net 15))
 (segment (start 100.877778 71.83502) (end 103.5558 69.156998) (width 0.25) (layer F.Cu) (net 15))
 (segment (start 100.965 68.4068) (end 103.5558 65.816) (width 0.25) (layer F.Cu) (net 35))
 (segment (start 100.965 71.111387) (end 100.965 68.4068) (width 0.25) (layer F.Cu) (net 35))
 (segment (start 100.427767 73.878835) (end 100.427767 71.64862) (width 0.25) (layer F.Cu) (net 35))
 (segment (start 95.256601 77.310999) (end 96.995603 77.310999) (width 0.25) (layer F.Cu) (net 35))
 (segment (start 94.0816 78.486) (end 95.256601 77.310999) (width 0.25) (layer F.Cu) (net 35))
 (segment (start 96.995603 77.310999) (end 100.427767 73.878835) (width 0.25) (layer F.Cu) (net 35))
 (segment (start 100.427767 71.64862) (end 100.965 71.111387) (width 0.25) (layer F.Cu) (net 35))
 (segment (start 99.977756 71.46222) (end 100.514989 70.924988) (width 0.25) (layer F.Cu) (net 16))
 (segment (start 100.514989 70.924988) (end 100.514989 68.176286) (width 0.25) (layer F.Cu) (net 16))
 (segment (start 100.514989 68.176286) (end 101.219475 67.471801) (width 0.25) (layer F.Cu) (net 16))
 (segment (start 96.6216 75.946) (end 99.977756 72.589844) (width 0.25) (layer F.Cu) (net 16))
 (segment (start 99.977756 72.589844) (end 99.977756 71.46222) (width 0.25) (layer F.Cu) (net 16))
 (segment (start 101.219475 67.471801) (end 101.219475 65.612324) (width 0.25) (layer F.Cu) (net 16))
 (segment (start 101.219475 65.612324) (end 103.5558 63.276) (width 0.25) (layer F.Cu) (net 16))
 (segment (start 100.769464 67.285401) (end 100.769464 63.522336) (width 0.25) (layer F.Cu) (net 36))
 (segment (start 100.769464 63.522336) (end 103.5558 60.736) (width 0.25) (layer F.Cu) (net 36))
 (segment (start 100.064978 70.738588) (end 100.064978 67.989886) (width 0.25) (layer F.Cu) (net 36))
 (segment (start 96.995603 74.770999) (end 99.527745 72.238857) (width 0.25) (layer F.Cu) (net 36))
 (segment (start 95.256601 74.770999) (end 96.995603 74.770999) (width 0.25) (layer F.Cu) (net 36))
 (segment (start 100.064978 67.989886) (end 100.769464 67.285401) (width 0.25) (layer F.Cu) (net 36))
 (segment (start 99.527745 72.238857) (end 99.527746 71.275819) (width 0.25) (layer F.Cu) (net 36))
 (segment (start 99.527746 71.275819) (end 100.064978 70.738588) (width 0.25) (layer F.Cu) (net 36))
 (segment (start 94.0816 75.946) (end 95.256601 74.770999) (width 0.25) (layer F.Cu) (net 36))
 (segment (start 100.319453 67.099001) (end 100.319453 63.335937) (width 0.25) (layer F.Cu) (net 17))
 (segment (start 102.380799 59.371001) (end 103.5558 58.196) (width 0.25) (layer F.Cu) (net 17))
 (segment (start 96.6216 73.406) (end 99.614967 70.412633) (width 0.25) (layer F.Cu) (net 17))
 (segment (start 100.319453 63.335937) (end 102.380799 61.274591) (width 0.25) (layer F.Cu) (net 17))
 (segment (start 99.614967 67.803486) (end 100.319453 67.099001) (width 0.25) (layer F.Cu) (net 17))
 (segment (start 99.614967 70.412633) (end 99.614967 67.803486) (width 0.25) (layer F.Cu) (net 17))
 (segment (start 102.380799 61.274591) (end 102.380799 59.371001) (width 0.25) (layer F.Cu) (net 17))
 (segment (start 95.256601 72.230999) (end 96.995603 72.230999) (width 0.25) (layer F.Cu) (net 37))
 (segment (start 101.930788 61.088191) (end 101.930788 57.281012) (width 0.25) (layer F.Cu) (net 37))
 (segment (start 96.995603 72.230999) (end 99.164956 70.061646) (width 0.25) (layer F.Cu) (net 37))
 (segment (start 99.164956 67.617086) (end 99.869442 66.912601) (width 0.25) (layer F.Cu) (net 37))
 (segment (start 99.164956 70.061646) (end 99.164956 67.617086) (width 0.25) (layer F.Cu) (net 37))
 (segment (start 99.869442 63.149537) (end 101.930788 61.088191) (width 0.25) (layer F.Cu) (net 37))
 (segment (start 94.0816 73.406) (end 95.256601 72.230999) (width 0.25) (layer F.Cu) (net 37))
 (segment (start 99.869442 66.912601) (end 99.869442 63.149537) (width 0.25) (layer F.Cu) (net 37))
 (segment (start 101.930788 57.281012) (end 103.5558 55.656) (width 0.25) (layer F.Cu) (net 37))
 (segment (start 96.6216 70.866) (end 98.714945 68.772655) (width 0.25) (layer F.Cu) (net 18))
 (segment (start 98.714945 68.772655) (end 98.714945 67.430686) (width 0.25) (layer F.Cu) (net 18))
 (segment (start 98.714945 67.430686) (end 99.419431 66.726201) (width 0.25) (layer F.Cu) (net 18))
 (segment (start 99.419431 66.726201) (end 99.419431 62.963137) (width 0.25) (layer F.Cu) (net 18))
 (segment (start 99.419431 62.963137) (end 101.480777 60.901791) (width 0.25) (layer F.Cu) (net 18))
 (segment (start 101.480777 60.901791) (end 101.480777 55.191023) (width 0.25) (layer F.Cu) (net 18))
 (segment (start 101.480777 55.191023) (end 102.705801 53.965999) (width 0.25) (layer F.Cu) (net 18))
 (segment (start 102.705801 53.965999) (end 103.5558 53.116) (width 0.25) (layer F.Cu) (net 18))
 (segment (start 97.141344 69.501001) (end 95.446599 69.501001) (width 0.25) (layer F.Cu) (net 38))
 (segment (start 98.96942 66.539801) (end 98.264934 67.244286) (width 0.25) (layer F.Cu) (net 38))
 (segment (start 95.446599 69.501001) (end 94.0816 70.866) (width 0.25) (layer F.Cu) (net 38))
 (segment (start 98.264934 67.244286) (end 98.264934 68.377412) (width 0.25) (layer F.Cu) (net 38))
 (segment (start 98.264934 68.377412) (end 97.141344 69.501001) (width 0.25) (layer F.Cu) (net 38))
 (segment (start 103.5558 50.576) (end 98.96942 55.16238) (width 0.25) (layer F.Cu) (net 38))
 (segment (start 98.96942 55.16238) (end 98.96942 66.539801) (width 0.25) (layer F.Cu) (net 38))
 (segment (start 103.5558 48.036) (end 98.519409 53.072391) (width 0.25) (layer F.Cu) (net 19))
 (segment (start 98.519409 53.072391) (end 98.519409 66.353401) (width 0.25) (layer F.Cu) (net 19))
 (segment (start 98.519409 66.353401) (end 96.6216 68.25121) (width 0.25) (layer F.Cu) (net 19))
 (segment (start 96.6216 68.25121) (end 96.6216 68.326) (width 0.25) (layer F.Cu) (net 19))
 (segment (start 94.0816 68.326) (end 95.0976 68.326) (width 0.25) (layer F.Cu) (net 39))
 (segment (start 95.0976 68.326) (end 95.0976 68.110998) (width 0.25) (layer F.Cu) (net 39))
 (segment (start 96.247597 66.961001) (end 97.275399 66.961001) (width 0.25) (layer F.Cu) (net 39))
 (segment (start 95.0976 68.110998) (end 96.247597 66.961001) (width 0.25) (layer F.Cu) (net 39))
 (segment (start 97.796601 51.255199) (end 103.5558 45.496) (width 0.25) (layer F.Cu) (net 39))
 (segment (start 97.796601 66.439799) (end 97.796601 51.255199) (width 0.25) (layer F.Cu) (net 39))
 (segment (start 97.275399 66.961001) (end 97.796601 66.439799) (width 0.25) (layer F.Cu) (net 39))
 (segment (start 103.5558 43.756998) (end 103.5558 42.956) (width 0.25) (layer F.Cu) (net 20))
 (segment (start 96.6216 50.691198) (end 103.5558 43.756998) (width 0.25) (layer F.Cu) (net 20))
 (segment (start 96.6216 65.786) (end 96.6216 50.691198) (width 0.25) (layer F.Cu) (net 20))
 (segment (start 94.0816 49.8902) (end 94.0816 65.786) (width 0.25) (layer F.Cu) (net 40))
 (segment (start 103.5558 40.416) (end 94.0816 49.8902) (width 0.25) (layer F.Cu) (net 40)))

